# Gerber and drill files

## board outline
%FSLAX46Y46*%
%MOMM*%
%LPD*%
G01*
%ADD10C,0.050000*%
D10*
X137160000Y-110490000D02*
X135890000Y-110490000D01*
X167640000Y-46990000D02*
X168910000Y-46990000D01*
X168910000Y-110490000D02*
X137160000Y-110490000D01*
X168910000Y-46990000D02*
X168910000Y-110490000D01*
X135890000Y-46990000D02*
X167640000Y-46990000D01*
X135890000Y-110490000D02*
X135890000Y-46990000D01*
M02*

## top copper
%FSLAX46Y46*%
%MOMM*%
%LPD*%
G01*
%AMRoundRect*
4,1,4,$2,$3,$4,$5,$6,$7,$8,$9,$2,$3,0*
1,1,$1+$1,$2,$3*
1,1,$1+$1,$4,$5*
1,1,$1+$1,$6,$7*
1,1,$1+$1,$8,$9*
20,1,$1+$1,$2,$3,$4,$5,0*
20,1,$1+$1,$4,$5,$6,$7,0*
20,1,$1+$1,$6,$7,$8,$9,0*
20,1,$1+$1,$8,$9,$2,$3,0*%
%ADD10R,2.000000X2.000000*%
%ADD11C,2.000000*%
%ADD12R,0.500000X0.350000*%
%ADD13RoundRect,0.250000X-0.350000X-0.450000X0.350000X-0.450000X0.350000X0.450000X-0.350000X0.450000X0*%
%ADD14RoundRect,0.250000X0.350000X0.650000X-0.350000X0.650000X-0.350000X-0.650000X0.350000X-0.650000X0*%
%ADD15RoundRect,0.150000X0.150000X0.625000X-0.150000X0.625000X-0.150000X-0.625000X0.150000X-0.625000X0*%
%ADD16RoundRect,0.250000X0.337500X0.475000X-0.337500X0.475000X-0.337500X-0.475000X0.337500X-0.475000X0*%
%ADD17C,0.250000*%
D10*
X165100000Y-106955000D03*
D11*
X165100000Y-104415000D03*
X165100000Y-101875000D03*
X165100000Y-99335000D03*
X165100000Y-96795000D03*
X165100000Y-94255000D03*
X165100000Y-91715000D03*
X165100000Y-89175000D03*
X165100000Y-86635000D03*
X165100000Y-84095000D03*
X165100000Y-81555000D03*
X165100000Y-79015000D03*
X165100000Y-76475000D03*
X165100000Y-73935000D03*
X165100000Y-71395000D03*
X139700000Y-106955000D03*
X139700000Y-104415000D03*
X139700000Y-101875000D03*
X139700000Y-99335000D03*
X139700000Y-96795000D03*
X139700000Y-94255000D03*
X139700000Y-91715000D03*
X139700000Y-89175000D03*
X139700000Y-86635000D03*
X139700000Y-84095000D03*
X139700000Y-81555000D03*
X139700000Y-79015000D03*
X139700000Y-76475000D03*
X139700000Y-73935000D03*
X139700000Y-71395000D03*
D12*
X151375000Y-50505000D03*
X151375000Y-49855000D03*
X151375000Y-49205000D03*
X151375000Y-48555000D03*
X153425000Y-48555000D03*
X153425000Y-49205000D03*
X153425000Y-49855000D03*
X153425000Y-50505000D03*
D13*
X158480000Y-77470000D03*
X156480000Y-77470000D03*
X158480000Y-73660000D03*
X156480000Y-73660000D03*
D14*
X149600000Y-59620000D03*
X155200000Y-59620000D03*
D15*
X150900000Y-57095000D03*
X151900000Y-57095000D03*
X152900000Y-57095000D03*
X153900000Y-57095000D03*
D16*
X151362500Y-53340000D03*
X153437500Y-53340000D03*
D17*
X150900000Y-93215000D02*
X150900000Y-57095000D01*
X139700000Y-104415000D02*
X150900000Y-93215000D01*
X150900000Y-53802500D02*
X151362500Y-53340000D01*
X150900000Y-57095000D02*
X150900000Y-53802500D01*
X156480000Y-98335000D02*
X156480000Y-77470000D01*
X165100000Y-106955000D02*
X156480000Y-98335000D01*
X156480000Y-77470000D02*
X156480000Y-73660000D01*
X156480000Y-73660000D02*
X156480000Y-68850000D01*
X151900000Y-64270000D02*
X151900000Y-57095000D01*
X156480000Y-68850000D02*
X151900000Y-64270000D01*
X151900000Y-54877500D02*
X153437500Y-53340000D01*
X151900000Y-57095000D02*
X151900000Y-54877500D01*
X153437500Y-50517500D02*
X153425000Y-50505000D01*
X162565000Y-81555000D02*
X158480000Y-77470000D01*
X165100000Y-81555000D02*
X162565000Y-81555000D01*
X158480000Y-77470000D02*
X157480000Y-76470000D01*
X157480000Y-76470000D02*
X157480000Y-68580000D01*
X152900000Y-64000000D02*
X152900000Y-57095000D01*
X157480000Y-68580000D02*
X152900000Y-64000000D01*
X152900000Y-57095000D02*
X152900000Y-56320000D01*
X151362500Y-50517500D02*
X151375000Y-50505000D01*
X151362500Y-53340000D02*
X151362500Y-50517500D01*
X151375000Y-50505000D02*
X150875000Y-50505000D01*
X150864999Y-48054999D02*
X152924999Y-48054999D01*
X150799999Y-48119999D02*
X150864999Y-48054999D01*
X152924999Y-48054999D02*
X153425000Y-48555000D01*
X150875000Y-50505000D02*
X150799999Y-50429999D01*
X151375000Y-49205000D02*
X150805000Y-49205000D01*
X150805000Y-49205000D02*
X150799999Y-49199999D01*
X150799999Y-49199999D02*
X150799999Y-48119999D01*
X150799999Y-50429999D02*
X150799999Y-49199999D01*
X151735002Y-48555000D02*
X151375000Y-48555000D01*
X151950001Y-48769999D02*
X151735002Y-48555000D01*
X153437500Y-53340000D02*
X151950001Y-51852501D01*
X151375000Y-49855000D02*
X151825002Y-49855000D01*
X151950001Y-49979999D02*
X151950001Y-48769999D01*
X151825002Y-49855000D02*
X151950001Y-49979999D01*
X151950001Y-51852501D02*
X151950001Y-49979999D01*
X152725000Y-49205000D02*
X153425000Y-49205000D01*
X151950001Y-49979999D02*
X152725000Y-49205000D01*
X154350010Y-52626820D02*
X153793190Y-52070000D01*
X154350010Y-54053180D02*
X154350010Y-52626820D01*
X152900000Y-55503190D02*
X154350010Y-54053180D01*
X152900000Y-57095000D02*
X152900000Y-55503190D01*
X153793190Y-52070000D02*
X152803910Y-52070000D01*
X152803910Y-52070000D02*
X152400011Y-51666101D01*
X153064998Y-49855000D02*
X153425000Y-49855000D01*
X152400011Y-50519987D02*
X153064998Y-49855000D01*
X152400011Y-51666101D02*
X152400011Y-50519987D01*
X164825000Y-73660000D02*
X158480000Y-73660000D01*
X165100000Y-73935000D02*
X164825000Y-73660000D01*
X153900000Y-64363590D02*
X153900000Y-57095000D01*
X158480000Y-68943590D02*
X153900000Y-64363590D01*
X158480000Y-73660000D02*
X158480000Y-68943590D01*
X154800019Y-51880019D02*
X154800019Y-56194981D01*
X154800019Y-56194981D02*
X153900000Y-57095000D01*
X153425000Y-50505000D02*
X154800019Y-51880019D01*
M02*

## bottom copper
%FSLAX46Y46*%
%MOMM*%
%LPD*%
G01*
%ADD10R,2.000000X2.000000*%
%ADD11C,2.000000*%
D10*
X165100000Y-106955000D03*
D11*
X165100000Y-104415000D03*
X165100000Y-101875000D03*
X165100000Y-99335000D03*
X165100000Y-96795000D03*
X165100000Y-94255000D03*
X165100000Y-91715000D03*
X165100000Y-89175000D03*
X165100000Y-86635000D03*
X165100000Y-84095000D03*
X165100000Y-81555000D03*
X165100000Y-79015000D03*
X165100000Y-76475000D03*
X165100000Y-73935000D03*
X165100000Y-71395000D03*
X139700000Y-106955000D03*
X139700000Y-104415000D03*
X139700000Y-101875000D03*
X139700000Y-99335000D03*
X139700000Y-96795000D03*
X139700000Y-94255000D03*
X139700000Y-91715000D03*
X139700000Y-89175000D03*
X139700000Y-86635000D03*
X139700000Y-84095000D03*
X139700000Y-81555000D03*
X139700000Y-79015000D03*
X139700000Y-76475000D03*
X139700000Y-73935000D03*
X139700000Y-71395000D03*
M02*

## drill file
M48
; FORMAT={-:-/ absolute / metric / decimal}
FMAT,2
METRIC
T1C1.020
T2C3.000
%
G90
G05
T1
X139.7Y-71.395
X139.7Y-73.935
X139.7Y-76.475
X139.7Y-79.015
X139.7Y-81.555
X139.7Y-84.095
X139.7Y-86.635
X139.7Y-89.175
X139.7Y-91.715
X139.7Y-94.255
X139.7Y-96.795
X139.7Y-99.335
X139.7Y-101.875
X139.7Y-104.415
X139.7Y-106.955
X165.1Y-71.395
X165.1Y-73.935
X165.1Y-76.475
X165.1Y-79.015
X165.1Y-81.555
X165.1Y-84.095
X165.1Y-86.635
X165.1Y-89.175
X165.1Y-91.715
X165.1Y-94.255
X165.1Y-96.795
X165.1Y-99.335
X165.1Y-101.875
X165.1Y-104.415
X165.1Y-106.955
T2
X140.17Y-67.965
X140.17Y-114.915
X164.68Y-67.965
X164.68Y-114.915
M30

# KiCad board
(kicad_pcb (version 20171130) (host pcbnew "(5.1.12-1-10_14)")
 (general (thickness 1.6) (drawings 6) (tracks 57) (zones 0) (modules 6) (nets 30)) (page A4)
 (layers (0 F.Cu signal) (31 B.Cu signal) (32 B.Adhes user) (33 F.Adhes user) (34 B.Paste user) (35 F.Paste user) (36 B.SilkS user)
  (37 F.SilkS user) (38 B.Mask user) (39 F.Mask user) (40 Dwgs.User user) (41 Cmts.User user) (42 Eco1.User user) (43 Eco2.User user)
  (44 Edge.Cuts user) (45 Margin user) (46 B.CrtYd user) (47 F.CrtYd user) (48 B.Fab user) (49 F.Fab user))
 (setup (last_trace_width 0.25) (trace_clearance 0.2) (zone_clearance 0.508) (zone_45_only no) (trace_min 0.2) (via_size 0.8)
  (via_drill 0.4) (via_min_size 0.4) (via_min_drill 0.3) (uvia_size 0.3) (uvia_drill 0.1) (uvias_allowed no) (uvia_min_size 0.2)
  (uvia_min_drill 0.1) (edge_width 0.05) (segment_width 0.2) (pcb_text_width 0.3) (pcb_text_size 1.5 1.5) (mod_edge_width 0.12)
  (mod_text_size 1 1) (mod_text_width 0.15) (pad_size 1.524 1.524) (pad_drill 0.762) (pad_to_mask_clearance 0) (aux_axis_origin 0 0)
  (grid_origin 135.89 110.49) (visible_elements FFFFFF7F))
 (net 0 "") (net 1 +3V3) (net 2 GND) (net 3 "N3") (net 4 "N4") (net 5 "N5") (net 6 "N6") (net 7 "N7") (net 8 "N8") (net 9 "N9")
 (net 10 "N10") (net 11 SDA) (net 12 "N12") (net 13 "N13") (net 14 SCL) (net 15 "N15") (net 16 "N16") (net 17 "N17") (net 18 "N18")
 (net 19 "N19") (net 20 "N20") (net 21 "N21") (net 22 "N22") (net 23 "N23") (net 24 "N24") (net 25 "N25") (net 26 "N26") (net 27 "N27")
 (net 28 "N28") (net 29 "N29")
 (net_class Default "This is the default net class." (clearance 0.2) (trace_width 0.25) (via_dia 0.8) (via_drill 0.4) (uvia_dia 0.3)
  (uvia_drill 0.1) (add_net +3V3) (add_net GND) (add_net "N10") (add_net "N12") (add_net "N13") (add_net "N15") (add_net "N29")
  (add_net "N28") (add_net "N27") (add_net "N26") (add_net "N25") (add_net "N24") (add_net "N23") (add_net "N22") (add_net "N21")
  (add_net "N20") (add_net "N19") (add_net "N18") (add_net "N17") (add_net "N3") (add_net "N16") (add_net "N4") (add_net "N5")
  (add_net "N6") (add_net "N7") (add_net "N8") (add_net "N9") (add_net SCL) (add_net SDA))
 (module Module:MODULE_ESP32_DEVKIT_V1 (layer F.Cu) (at 152.4 91.44 180)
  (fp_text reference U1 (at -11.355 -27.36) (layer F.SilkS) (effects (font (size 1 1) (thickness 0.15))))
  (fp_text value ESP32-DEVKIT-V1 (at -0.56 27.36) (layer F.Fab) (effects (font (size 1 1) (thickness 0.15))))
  (pad 1 thru_hole rect (at -12.7 -15.515 180) (size 2 2) (drill 1.02) (layers *.Cu *.Mask) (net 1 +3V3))
  (pad 2 thru_hole circle (at -12.7 -12.975 180) (size 2 2) (drill 1.02) (layers *.Cu *.Mask) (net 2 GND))
  (pad 3 thru_hole circle (at -12.7 -10.435 180) (size 2 2) (drill 1.02) (layers *.Cu *.Mask) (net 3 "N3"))
  (pad 4 thru_hole circle (at -12.7 -7.895 180) (size 2 2) (drill 1.02) (layers *.Cu *.Mask) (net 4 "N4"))
  (pad 5 thru_hole circle (at -12.7 -5.355 180) (size 2 2) (drill 1.02) (layers *.Cu *.Mask) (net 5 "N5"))
  (pad 6 thru_hole circle (at -12.7 -2.815 180) (size 2 2) (drill 1.02) (layers *.Cu *.Mask) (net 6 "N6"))
  (pad 7 thru_hole circle (at -12.7 -0.275 180) (size 2 2) (drill 1.02) (layers *.Cu *.Mask) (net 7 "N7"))
  (pad 8 thru_hole circle (at -12.7 2.265 180) (size 2 2) (drill 1.02) (layers *.Cu *.Mask) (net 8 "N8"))
  (pad 9 thru_hole circle (at -12.7 4.805 180) (size 2 2) (drill 1.02) (layers *.Cu *.Mask) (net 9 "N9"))
  (pad 10 thru_hole circle (at -12.7 7.345 180) (size 2 2) (drill 1.02) (layers *.Cu *.Mask) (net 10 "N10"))
  (pad 11 thru_hole circle (at -12.7 9.885 180) (size 2 2) (drill 1.02) (layers *.Cu *.Mask) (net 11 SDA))
  (pad 12 thru_hole circle (at -12.7 12.425 180) (size 2 2) (drill 1.02) (layers *.Cu *.Mask) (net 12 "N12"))
  (pad 13 thru_hole circle (at -12.7 14.965 180) (size 2 2) (drill 1.02) (layers *.Cu *.Mask) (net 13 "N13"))
  (pad 14 thru_hole circle (at -12.7 17.505 180) (size 2 2) (drill 1.02) (layers *.Cu *.Mask) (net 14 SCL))
  (pad 15 thru_hole circle (at -12.7 20.045 180) (size 2 2) (drill 1.02) (layers *.Cu *.Mask) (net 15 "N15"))
  (pad 30 thru_hole circle (at 12.7 -15.515 180) (size 2 2) (drill 1.02) (layers *.Cu *.Mask) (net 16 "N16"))
  (pad 29 thru_hole circle (at 12.7 -12.975 180) (size 2 2) (drill 1.02) (layers *.Cu *.Mask) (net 2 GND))
  (pad 28 thru_hole circle (at 12.7 -10.435 180) (size 2 2) (drill 1.02) (layers *.Cu *.Mask) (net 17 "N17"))
  (pad 27 thru_hole circle (at 12.7 -7.895 180) (size 2 2) (drill 1.02) (layers *.Cu *.Mask) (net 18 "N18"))
  (pad 26 thru_hole circle (at 12.7 -5.355 180) (size 2 2) (drill 1.02) (layers *.Cu *.Mask) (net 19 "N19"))
  (pad 25 thru_hole circle (at 12.7 -2.815 180) (size 2 2) (drill 1.02) (layers *.Cu *.Mask) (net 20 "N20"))
  (pad 24 thru_hole circle (at 12.7 -0.275 180) (size 2 2) (drill 1.02) (layers *.Cu *.Mask) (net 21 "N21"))
  (pad 23 thru_hole circle (at 12.7 2.265 180) (size 2 2) (drill 1.02) (layers *.Cu *.Mask) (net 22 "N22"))
  (pad 22 thru_hole circle (at 12.7 4.805 180) (size 2 2) (drill 1.02) (layers *.Cu *.Mask) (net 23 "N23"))
  (pad 21 thru_hole circle (at 12.7 7.345 180) (size 2 2) (drill 1.02) (layers *.Cu *.Mask) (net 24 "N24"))
  (pad 20 thru_hole circle (at 12.7 9.885 180) (size 2 2) (drill 1.02) (layers *.Cu *.Mask) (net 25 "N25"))
  (pad 19 thru_hole circle (at 12.7 12.425 180) (size 2 2) (drill 1.02) (layers *.Cu *.Mask) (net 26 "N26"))
  (pad 18 thru_hole circle (at 12.7 14.965 180) (size 2 2) (drill 1.02) (layers *.Cu *.Mask) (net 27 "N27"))
  (pad 17 thru_hole circle (at 12.7 17.505 180) (size 2 2) (drill 1.02) (layers *.Cu *.Mask) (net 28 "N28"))
  (pad 16 thru_hole circle (at 12.7 20.045 180) (size 2 2) (drill 1.02) (layers *.Cu *.Mask) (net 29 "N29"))
  (pad None np_thru_hole circle (at -12.28 23.475 180) (size 3 3) (drill 3) (layers *.Cu *.Mask))
  (pad None np_thru_hole circle (at 12.23 23.475 180) (size 3 3) (drill 3) (layers *.Cu *.Mask))
  (pad None np_thru_hole circle (at 12.23 -23.475 180) (size 3 3) (drill 3) (layers *.Cu *.Mask))
  (pad None np_thru_hole circle (at -12.28 -23.475 180) (size 3 3) (drill 3) (layers *.Cu *.Mask)))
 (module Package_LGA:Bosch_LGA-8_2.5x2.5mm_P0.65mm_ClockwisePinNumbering (layer F.Cu) (at 152.4 49.53 270)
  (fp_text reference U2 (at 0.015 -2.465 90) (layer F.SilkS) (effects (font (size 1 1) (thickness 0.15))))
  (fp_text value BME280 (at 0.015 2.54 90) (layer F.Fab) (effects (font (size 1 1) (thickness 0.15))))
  (pad 5 smd rect (at 0.975 1.025) (size 0.5 0.35) (layers F.Cu F.Paste F.Mask) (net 2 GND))
  (pad 6 smd rect (at 0.325 1.025) (size 0.5 0.35) (layers F.Cu F.Paste F.Mask) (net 1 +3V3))
  (pad 7 smd rect (at -0.325 1.025) (size 0.5 0.35) (layers F.Cu F.Paste F.Mask) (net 2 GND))
  (pad 8 smd rect (at -0.975 1.025) (size 0.5 0.35) (layers F.Cu F.Paste F.Mask) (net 1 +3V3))
  (pad 1 smd rect (at -0.975 -1.025) (size 0.5 0.35) (layers F.Cu F.Paste F.Mask) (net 2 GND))
  (pad 2 smd rect (at -0.325 -1.025) (size 0.5 0.35) (layers F.Cu F.Paste F.Mask) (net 1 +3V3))
  (pad 3 smd rect (at 0.325 -1.025) (size 0.5 0.35) (layers F.Cu F.Paste F.Mask) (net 11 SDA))
  (pad 4 smd rect (at 0.975 -1.025) (size 0.5 0.35) (layers F.Cu F.Paste F.Mask) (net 14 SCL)))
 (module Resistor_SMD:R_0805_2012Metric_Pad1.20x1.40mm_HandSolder (layer F.Cu) (at 157.48 77.47)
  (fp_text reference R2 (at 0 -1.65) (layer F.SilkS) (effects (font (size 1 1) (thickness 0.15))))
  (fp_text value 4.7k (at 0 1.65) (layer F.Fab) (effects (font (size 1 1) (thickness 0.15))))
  (pad 2 smd roundrect (at 1 0) (size 1.2 1.4) (layers F.Cu F.Paste F.Mask) (roundrect_rratio 0.208333) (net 11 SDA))
  (pad 1 smd roundrect (at -1 0) (size 1.2 1.4) (layers F.Cu F.Paste F.Mask) (roundrect_rratio 0.208333) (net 1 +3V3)))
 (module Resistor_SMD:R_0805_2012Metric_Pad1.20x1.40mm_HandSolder (layer F.Cu) (at 157.48 73.66)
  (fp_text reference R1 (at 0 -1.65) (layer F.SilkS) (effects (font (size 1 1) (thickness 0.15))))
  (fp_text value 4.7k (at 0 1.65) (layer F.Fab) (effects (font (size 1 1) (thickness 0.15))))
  (pad 2 smd roundrect (at 1 0) (size 1.2 1.4) (layers F.Cu F.Paste F.Mask) (roundrect_rratio 0.208333) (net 14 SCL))
  (pad 1 smd roundrect (at -1 0) (size 1.2 1.4) (layers F.Cu F.Paste F.Mask) (roundrect_rratio 0.208333) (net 1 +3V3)))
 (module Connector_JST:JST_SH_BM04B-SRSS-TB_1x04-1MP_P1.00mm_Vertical (layer F.Cu) (at 152.4 58.42 180)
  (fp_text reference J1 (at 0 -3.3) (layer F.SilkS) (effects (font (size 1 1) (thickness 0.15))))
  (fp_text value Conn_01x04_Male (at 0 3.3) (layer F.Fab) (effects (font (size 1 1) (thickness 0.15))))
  (pad MP smd roundrect (at 2.8 -1.2 180) (size 1.2 1.8) (layers F.Cu F.Paste F.Mask) (roundrect_rratio 0.208333))
  (pad MP smd roundrect (at -2.8 -1.2 180) (size 1.2 1.8) (layers F.Cu F.Paste F.Mask) (roundrect_rratio 0.208333))
  (pad 4 smd roundrect (at 1.5 1.325 180) (size 0.6 1.55) (layers F.Cu F.Paste F.Mask) (roundrect_rratio 0.25) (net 2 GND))
  (pad 3 smd roundrect (at 0.5 1.325 180) (size 0.6 1.55) (layers F.Cu F.Paste F.Mask) (roundrect_rratio 0.25) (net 1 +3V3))
  (pad 2 smd roundrect (at -0.5 1.325 180) (size 0.6 1.55) (layers F.Cu F.Paste F.Mask) (roundrect_rratio 0.25) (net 11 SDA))
  (pad 1 smd roundrect (at -1.5 1.325 180) (size 0.6 1.55) (layers F.Cu F.Paste F.Mask) (roundrect_rratio 0.25) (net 14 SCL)))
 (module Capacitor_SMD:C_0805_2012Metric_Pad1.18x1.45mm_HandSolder (layer F.Cu) (at 152.4 53.34 180)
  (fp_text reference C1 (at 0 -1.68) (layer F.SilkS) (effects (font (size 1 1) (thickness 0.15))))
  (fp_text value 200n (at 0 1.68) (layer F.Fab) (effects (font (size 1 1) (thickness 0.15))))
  (pad 2 smd roundrect (at 1.0375 0 180) (size 1.175 1.45) (layers F.Cu F.Paste F.Mask) (roundrect_rratio 0.212766) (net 2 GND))
  (pad 1 smd roundrect (at -1.0375 0 180) (size 1.175 1.45) (layers F.Cu F.Paste F.Mask) (roundrect_rratio 0.212766) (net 1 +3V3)))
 (gr_line (start 137.16 110.49) (end 135.89 110.49) (layer Edge.Cuts) (width 0.05))
 (gr_line (start 167.64 46.99) (end 168.91 46.99) (layer Edge.Cuts) (width 0.05))
 (gr_line (start 168.91 110.49) (end 137.16 110.49) (layer Edge.Cuts) (width 0.05))
 (gr_line (start 168.91 46.99) (end 168.91 110.49) (layer Edge.Cuts) (width 0.05))
 (gr_line (start 135.89 46.99) (end 167.64 46.99) (layer Edge.Cuts) (width 0.05))
 (gr_line (start 135.89 110.49) (end 135.89 46.99) (layer Edge.Cuts) (width 0.05))
 (segment (start 150.9 93.215) (end 150.9 57.095) (width 0.25) (layer F.Cu) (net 2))
 (segment (start 139.7 104.415) (end 150.9 93.215) (width 0.25) (layer F.Cu) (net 2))
 (segment (start 150.9 53.8025) (end 151.3625 53.34) (width 0.25) (layer F.Cu) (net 2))
 (segment (start 150.9 57.095) (end 150.9 53.8025) (width 0.25) (layer F.Cu) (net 2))
 (segment (start 156.48 98.335) (end 156.48 77.47) (width 0.25) (layer F.Cu) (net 1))
 (segment (start 165.1 106.955) (end 156.48 98.335) (width 0.25) (layer F.Cu) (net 1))
 (segment (start 156.48 77.47) (end 156.48 73.66) (width 0.25) (layer F.Cu) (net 1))
 (segment (start 156.48 73.66) (end 156.48 68.85) (width 0.25) (layer F.Cu) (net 1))
 (segment (start 151.9 64.27) (end 151.9 57.095) (width 0.25) (layer F.Cu) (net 1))
 (segment (start 156.48 68.85) (end 151.9 64.27) (width 0.25) (layer F.Cu) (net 1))
 (segment (start 151.9 54.8775) (end 153.4375 53.34) (width 0.25) (layer F.Cu) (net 1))
 (segment (start 151.9 57.095) (end 151.9 54.8775) (width 0.25) (layer F.Cu) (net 1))
 (segment (start 153.4375 50.5175) (end 153.425 50.505) (width 0.25) (layer F.Cu) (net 14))
 (segment (start 162.565 81.555) (end 158.48 77.47) (width 0.25) (layer F.Cu) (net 11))
 (segment (start 165.1 81.555) (end 162.565 81.555) (width 0.25) (layer F.Cu) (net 11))
 (segment (start 158.48 77.47) (end 157.48 76.47) (width 0.25) (layer F.Cu) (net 11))
 (segment (start 157.48 76.47) (end 157.48 68.58) (width 0.25) (layer F.Cu) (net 11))
 (segment (start 152.9 64) (end 152.9 57.095) (width 0.25) (layer F.Cu) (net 11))
 (segment (start 157.48 68.58) (end 152.9 64) (width 0.25) (layer F.Cu) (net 11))
 (segment (start 152.9 57.095) (end 152.9 56.32) (width 0.25) (layer F.Cu) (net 11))
 (segment (start 151.3625 50.5175) (end 151.375 50.505) (width 0.25) (layer F.Cu) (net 2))
 (segment (start 151.3625 53.34) (end 151.3625 50.5175) (width 0.25) (layer F.Cu) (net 2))
 (segment (start 151.375 50.505) (end 150.875 50.505) (width 0.25) (layer F.Cu) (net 2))
 (segment (start 150.864999 48.054999) (end 152.924999 48.054999) (width 0.25) (layer F.Cu) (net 2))
 (segment (start 150.799999 48.119999) (end 150.864999 48.054999) (width 0.25) (layer F.Cu) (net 2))
 (segment (start 152.924999 48.054999) (end 153.425 48.555) (width 0.25) (layer F.Cu) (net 2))
 (segment (start 150.875 50.505) (end 150.799999 50.429999) (width 0.25) (layer F.Cu) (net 2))
 (segment (start 151.375 49.205) (end 150.805 49.205) (width 0.25) (layer F.Cu) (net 2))
 (segment (start 150.805 49.205) (end 150.799999 49.199999) (width 0.25) (layer F.Cu) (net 2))
 (segment (start 150.799999 49.199999) (end 150.799999 48.119999) (width 0.25) (layer F.Cu) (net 2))
 (segment (start 150.799999 50.429999) (end 150.799999 49.199999) (width 0.25) (layer F.Cu) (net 2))
 (segment (start 151.735002 48.555) (end 151.375 48.555) (width 0.25) (layer F.Cu) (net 1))
 (segment (start 151.950001 48.769999) (end 151.735002 48.555) (width 0.25) (layer F.Cu) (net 1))
 (segment (start 153.4375 53.34) (end 151.950001 51.852501) (width 0.25) (layer F.Cu) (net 1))
 (segment (start 151.375 49.855) (end 151.825002 49.855) (width 0.25) (layer F.Cu) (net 1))
 (segment (start 151.950001 49.979999) (end 151.950001 48.769999) (width 0.25) (layer F.Cu) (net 1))
 (segment (start 151.825002 49.855) (end 151.950001 49.979999) (width 0.25) (layer F.Cu) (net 1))
 (segment (start 151.950001 51.852501) (end 151.950001 49.979999) (width 0.25) (layer F.Cu) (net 1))
 (segment (start 152.725 49.205) (end 153.425 49.205) (width 0.25) (layer F.Cu) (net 1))
 (segment (start 151.950001 49.979999) (end 152.725 49.205) (width 0.25) (layer F.Cu) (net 1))
 (segment (start 154.35001 52.62682) (end 153.79319 52.07) (width 0.25) (layer F.Cu) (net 11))
 (segment (start 154.35001 54.05318) (end 154.35001 52.62682) (width 0.25) (layer F.Cu) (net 11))
 (segment (start 152.9 55.50319) (end 154.35001 54.05318) (width 0.25) (layer F.Cu) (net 11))
 (segment (start 152.9 57.095) (end 152.9 55.50319) (width 0.25) (layer F.Cu) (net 11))
 (segment (start 153.79319 52.07) (end 152.80391 52.07) (width 0.25) (layer F.Cu) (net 11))
 (segment (start 152.80391 52.07) (end 152.400011 51.666101) (width 0.25) (layer F.Cu) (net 11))
 (segment (start 153.064998 49.855) (end 153.425 49.855) (width 0.25) (layer F.Cu) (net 11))
 (segment (start 152.400011 50.519987) (end 153.064998 49.855) (width 0.25) (layer F.Cu) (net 11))
 (segment (start 152.400011 51.666101) (end 152.400011 50.519987) (width 0.25) (layer F.Cu) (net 11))
 (segment (start 164.825 73.66) (end 158.48 73.66) (width 0.25) (layer F.Cu) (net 14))
 (segment (start 165.1 73.935) (end 164.825 73.66) (width 0.25) (layer F.Cu) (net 14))
 (segment (start 153.9 64.36359) (end 153.9 57.095) (width 0.25) (layer F.Cu) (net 14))
 (segment (start 158.48 68.94359) (end 153.9 64.36359) (width 0.25) (layer F.Cu) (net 14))
 (segment (start 158.48 73.66) (end 158.48 68.94359) (width 0.25) (layer F.Cu) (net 14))
 (segment (start 154.800019 51.880019) (end 154.800019 56.194981) (width 0.25) (layer F.Cu) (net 14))
 (segment (start 154.800019 56.194981) (end 153.9 57.095) (width 0.25) (layer F.Cu) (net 14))
 (segment (start 153.425 50.505) (end 154.800019 51.880019) (width 0.25) (layer F.Cu) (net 14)))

